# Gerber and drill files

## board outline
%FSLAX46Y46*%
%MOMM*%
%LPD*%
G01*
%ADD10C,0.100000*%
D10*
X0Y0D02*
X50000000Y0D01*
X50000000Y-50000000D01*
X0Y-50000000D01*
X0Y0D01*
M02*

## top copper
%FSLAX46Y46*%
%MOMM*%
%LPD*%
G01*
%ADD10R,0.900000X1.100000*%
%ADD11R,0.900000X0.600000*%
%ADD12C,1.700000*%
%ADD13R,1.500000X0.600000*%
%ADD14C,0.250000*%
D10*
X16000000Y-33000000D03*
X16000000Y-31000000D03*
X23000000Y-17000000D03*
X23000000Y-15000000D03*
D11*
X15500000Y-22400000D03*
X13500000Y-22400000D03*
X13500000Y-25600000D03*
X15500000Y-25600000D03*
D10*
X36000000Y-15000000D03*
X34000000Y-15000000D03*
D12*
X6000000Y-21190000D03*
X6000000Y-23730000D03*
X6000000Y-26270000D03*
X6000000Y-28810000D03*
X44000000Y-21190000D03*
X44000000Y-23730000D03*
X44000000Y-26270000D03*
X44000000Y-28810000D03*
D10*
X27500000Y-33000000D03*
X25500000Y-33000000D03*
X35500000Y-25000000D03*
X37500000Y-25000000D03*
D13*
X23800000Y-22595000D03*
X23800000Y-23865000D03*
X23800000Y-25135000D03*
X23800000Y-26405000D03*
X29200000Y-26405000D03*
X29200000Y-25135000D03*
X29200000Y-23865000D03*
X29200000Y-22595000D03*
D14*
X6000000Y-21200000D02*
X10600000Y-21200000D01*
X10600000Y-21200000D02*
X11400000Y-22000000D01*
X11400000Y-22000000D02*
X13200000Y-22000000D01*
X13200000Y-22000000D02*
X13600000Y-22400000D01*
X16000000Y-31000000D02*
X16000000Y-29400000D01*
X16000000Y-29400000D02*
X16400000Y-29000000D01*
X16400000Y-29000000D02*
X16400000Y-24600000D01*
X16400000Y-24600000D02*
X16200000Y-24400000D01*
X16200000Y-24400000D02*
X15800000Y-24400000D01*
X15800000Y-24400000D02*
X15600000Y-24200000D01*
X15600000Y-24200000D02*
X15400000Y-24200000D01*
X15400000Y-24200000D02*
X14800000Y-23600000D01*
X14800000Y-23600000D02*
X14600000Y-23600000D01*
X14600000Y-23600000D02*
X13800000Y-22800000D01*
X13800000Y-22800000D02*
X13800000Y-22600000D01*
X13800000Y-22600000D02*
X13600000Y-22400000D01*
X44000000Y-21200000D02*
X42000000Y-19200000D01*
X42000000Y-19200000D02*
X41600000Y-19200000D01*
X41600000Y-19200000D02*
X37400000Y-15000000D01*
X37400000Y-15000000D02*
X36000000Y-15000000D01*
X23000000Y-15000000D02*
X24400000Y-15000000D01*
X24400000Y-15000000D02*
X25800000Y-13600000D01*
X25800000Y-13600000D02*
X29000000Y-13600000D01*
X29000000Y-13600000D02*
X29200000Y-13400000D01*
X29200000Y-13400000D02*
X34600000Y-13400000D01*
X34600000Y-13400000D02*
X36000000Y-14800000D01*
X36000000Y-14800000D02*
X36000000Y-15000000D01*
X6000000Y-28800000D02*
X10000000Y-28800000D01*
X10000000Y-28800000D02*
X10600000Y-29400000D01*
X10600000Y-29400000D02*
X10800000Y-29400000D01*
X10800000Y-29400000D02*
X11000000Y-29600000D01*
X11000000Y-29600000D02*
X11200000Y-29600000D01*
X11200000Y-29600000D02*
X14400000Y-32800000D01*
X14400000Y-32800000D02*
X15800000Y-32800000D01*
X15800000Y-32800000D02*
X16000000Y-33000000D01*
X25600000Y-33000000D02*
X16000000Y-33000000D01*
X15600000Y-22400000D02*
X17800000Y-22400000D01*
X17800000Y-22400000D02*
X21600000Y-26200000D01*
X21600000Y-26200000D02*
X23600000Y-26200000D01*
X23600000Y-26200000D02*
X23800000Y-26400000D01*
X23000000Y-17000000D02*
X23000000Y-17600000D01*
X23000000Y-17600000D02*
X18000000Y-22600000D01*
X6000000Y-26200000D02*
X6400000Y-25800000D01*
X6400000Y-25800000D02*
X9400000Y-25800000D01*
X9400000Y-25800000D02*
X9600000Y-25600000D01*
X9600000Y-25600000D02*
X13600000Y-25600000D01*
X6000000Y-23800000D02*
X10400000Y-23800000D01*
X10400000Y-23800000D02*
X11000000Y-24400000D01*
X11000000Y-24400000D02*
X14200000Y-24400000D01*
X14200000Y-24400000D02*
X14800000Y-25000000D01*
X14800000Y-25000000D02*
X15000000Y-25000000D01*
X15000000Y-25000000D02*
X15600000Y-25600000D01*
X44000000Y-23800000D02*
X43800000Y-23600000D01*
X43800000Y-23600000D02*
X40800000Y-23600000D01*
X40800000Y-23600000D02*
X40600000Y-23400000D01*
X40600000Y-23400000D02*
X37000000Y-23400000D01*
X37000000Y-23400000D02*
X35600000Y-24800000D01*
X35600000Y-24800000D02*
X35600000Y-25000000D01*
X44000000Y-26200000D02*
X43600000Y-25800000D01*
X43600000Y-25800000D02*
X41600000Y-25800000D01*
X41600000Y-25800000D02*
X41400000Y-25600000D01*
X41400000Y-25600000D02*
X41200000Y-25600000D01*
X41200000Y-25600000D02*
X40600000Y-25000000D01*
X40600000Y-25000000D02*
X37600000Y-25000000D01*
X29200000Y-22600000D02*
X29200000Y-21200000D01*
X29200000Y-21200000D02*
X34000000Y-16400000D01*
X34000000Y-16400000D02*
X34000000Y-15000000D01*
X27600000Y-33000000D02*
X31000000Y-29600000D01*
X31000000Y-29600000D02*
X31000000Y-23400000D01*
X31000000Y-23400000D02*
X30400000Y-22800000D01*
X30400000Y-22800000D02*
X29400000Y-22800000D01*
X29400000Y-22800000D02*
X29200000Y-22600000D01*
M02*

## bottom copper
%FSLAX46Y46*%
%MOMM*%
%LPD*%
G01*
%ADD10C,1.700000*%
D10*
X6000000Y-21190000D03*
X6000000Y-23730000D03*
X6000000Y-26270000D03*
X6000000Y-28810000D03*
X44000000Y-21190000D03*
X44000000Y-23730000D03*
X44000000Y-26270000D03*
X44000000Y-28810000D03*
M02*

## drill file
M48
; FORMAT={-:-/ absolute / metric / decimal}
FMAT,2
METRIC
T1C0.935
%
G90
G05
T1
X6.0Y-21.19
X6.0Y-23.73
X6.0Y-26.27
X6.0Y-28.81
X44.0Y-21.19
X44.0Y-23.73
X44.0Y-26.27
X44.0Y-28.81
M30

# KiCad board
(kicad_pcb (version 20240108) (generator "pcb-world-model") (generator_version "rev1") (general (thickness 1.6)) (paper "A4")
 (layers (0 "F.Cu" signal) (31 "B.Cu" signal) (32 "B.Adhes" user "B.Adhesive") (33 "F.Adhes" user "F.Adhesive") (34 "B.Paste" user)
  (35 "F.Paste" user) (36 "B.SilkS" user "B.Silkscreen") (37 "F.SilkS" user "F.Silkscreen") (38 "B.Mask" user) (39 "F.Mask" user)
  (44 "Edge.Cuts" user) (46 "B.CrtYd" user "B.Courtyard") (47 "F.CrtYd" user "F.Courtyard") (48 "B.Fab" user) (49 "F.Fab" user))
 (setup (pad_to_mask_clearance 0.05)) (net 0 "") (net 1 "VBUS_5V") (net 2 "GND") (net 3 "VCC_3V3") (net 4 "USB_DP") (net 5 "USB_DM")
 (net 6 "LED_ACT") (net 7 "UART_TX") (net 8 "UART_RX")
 (gr_rect (start 0.0 0.0) (end 50.0000 50.0000) (stroke (width 0.1) (type default)) (fill none) (layer "Edge.Cuts"))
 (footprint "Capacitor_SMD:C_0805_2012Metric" (layer "F.Cu") (at 16.0000 32.0000 90)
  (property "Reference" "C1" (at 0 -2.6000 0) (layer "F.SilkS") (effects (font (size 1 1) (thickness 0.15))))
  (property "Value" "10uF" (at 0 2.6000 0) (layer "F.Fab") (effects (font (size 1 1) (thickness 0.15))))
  (pad "1" smd rect (at -1.0000 0.0000) (size 0.9000 1.1000) (layers "F.Cu" "F.Paste" "F.Mask") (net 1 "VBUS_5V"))
  (pad "2" smd rect (at 1.0000 0.0000) (size 0.9000 1.1000) (layers "F.Cu" "F.Paste" "F.Mask") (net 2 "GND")))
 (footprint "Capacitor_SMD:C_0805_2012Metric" (layer "F.Cu") (at 23.0000 16.0000 90)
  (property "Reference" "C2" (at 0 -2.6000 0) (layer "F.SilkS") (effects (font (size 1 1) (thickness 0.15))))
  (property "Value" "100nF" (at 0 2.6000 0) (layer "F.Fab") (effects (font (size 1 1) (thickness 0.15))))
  (pad "1" smd rect (at -1.0000 0.0000) (size 0.9000 1.1000) (layers "F.Cu" "F.Paste" "F.Mask") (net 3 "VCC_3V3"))
  (pad "2" smd rect (at 1.0000 0.0000) (size 0.9000 1.1000) (layers "F.Cu" "F.Paste" "F.Mask") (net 2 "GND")))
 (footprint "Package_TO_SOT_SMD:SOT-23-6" (layer "F.Cu") (at 14.5000 24.0000 270)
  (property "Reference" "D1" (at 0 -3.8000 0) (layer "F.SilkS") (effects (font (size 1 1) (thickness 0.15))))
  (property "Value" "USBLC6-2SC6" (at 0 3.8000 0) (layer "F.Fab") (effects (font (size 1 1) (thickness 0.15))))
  (pad "1" smd rect (at -1.6000 -1.0000) (size 0.9000 0.6000) (layers "F.Cu" "F.Paste" "F.Mask") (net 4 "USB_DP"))
  (pad "2" smd rect (at -1.6000 1.0000) (size 0.9000 0.6000) (layers "F.Cu" "F.Paste" "F.Mask") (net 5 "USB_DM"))
  (pad "3" smd rect (at 1.6000 1.0000) (size 0.9000 0.6000) (layers "F.Cu" "F.Paste" "F.Mask") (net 2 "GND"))
  (pad "4" smd rect (at 1.6000 -1.0000) (size 0.9000 0.6000) (layers "F.Cu" "F.Paste" "F.Mask") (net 1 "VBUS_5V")))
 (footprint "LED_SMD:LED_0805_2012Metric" (layer "F.Cu") (at 35.0000 15.0000 180)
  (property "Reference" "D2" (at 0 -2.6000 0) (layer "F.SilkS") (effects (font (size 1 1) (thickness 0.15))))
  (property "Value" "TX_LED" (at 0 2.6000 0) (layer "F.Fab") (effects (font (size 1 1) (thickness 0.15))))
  (pad "1" smd rect (at -1.0000 0.0000) (size 0.9000 1.1000) (layers "F.Cu" "F.Paste" "F.Mask") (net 3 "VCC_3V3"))
  (pad "2" smd rect (at 1.0000 0.0000) (size 0.9000 1.1000) (layers "F.Cu" "F.Paste" "F.Mask") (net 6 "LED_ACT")))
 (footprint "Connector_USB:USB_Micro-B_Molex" (layer "F.Cu") (at 6.0000 25.0000 0) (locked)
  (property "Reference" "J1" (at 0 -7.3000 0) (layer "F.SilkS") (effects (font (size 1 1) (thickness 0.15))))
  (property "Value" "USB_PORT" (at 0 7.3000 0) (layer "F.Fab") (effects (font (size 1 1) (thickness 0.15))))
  (pad "1" thru_hole circle (at 0.0000 -3.8100) (size 1.7000 1.7000) (drill 0.9350) (layers "*.Cu" "*.Mask") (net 1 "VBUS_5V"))
  (pad "2" thru_hole circle (at 0.0000 -1.2700) (size 1.7000 1.7000) (drill 0.9350) (layers "*.Cu" "*.Mask") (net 5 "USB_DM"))
  (pad "3" thru_hole circle (at 0.0000 1.2700) (size 1.7000 1.7000) (drill 0.9350) (layers "*.Cu" "*.Mask") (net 4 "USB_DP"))
  (pad "4" thru_hole circle (at 0.0000 3.8100) (size 1.7000 1.7000) (drill 0.9350) (layers "*.Cu" "*.Mask") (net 2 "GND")))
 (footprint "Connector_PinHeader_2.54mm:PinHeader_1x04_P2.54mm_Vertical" (layer "F.Cu") (at 44.0000 25.0000 0) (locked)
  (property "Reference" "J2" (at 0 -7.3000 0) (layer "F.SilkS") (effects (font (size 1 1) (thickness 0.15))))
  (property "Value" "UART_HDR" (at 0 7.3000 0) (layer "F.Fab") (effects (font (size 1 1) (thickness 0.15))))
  (pad "1" thru_hole circle (at 0.0000 -3.8100) (size 1.7000 1.7000) (drill 0.9350) (layers "*.Cu" "*.Mask") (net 3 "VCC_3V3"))
  (pad "2" thru_hole circle (at 0.0000 -1.2700) (size 1.7000 1.7000) (drill 0.9350) (layers "*.Cu" "*.Mask") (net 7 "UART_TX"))
  (pad "3" thru_hole circle (at 0.0000 1.2700) (size 1.7000 1.7000) (drill 0.9350) (layers "*.Cu" "*.Mask") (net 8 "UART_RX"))
  (pad "4" thru_hole circle (at 0.0000 3.8100) (size 1.7000 1.7000) (drill 0.9350) (layers "*.Cu" "*.Mask") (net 2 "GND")))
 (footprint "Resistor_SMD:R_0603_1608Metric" (layer "F.Cu") (at 26.5000 33.0000 180)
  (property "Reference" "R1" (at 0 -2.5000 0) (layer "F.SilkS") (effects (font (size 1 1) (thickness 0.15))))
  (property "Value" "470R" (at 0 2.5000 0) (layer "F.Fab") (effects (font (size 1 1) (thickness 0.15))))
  (pad "1" smd rect (at -1.0000 0.0000) (size 0.9000 1.1000) (layers "F.Cu" "F.Paste" "F.Mask") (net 6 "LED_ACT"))
  (pad "2" smd rect (at 1.0000 0.0000) (size 0.9000 1.1000) (layers "F.Cu" "F.Paste" "F.Mask") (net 2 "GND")))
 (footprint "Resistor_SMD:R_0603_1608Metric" (layer "F.Cu") (at 36.5000 25.0000 0)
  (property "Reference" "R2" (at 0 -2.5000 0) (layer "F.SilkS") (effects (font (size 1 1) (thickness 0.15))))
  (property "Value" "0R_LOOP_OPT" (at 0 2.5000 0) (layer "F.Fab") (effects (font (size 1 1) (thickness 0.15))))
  (pad "1" smd rect (at -1.0000 0.0000) (size 0.9000 1.1000) (layers "F.Cu" "F.Paste" "F.Mask") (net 7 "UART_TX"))
  (pad "2" smd rect (at 1.0000 0.0000) (size 0.9000 1.1000) (layers "F.Cu" "F.Paste" "F.Mask") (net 8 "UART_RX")))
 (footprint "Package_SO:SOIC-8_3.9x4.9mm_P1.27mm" (layer "F.Cu") (at 26.5000 24.5000 0)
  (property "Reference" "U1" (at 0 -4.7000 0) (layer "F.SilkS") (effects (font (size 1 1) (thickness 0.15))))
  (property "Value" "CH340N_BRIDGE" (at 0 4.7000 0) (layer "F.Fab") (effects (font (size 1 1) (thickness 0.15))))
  (pad "1" smd rect (at -2.7000 -1.9050) (size 1.5000 0.6000) (layers "F.Cu" "F.Paste" "F.Mask") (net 1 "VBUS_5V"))
  (pad "2" smd rect (at -2.7000 -0.6350) (size 1.5000 0.6000) (layers "F.Cu" "F.Paste" "F.Mask") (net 4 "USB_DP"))
  (pad "3" smd rect (at -2.7000 0.6350) (size 1.5000 0.6000) (layers "F.Cu" "F.Paste" "F.Mask") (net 5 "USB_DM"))
  (pad "4" smd rect (at -2.7000 1.9050) (size 1.5000 0.6000) (layers "F.Cu" "F.Paste" "F.Mask") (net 2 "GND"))
  (pad "5" smd rect (at 2.7000 1.9050) (size 1.5000 0.6000) (layers "F.Cu" "F.Paste" "F.Mask") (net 3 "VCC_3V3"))
  (pad "6" smd rect (at 2.7000 0.6350) (size 1.5000 0.6000) (layers "F.Cu" "F.Paste" "F.Mask") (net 7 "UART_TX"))
  (pad "7" smd rect (at 2.7000 -0.6350) (size 1.5000 0.6000) (layers "F.Cu" "F.Paste" "F.Mask") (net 8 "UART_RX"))
  (pad "8" smd rect (at 2.7000 -1.9050) (size 1.5000 0.6000) (layers "F.Cu" "F.Paste" "F.Mask") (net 6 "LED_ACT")))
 (segment (start 6.0000 21.2000) (end 10.6000 21.2000) (width 0.2500) (layer "F.Cu") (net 1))
 (segment (start 10.6000 21.2000) (end 11.4000 22.0000) (width 0.2500) (layer "F.Cu") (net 1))
 (segment (start 11.4000 22.0000) (end 13.2000 22.0000) (width 0.2500) (layer "F.Cu") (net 1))
 (segment (start 13.2000 22.0000) (end 13.6000 22.4000) (width 0.2500) (layer "F.Cu") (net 1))
 (segment (start 16.0000 31.0000) (end 16.0000 29.4000) (width 0.2500) (layer "F.Cu") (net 1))
 (segment (start 16.0000 29.4000) (end 16.4000 29.0000) (width 0.2500) (layer "F.Cu") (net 1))
 (segment (start 16.4000 29.0000) (end 16.4000 24.6000) (width 0.2500) (layer "F.Cu") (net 1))
 (segment (start 16.4000 24.6000) (end 16.2000 24.4000) (width 0.2500) (layer "F.Cu") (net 1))
 (segment (start 16.2000 24.4000) (end 15.8000 24.4000) (width 0.2500) (layer "F.Cu") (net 1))
 (segment (start 15.8000 24.4000) (end 15.6000 24.2000) (width 0.2500) (layer "F.Cu") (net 1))
 (segment (start 15.6000 24.2000) (end 15.4000 24.2000) (width 0.2500) (layer "F.Cu") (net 1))
 (segment (start 15.4000 24.2000) (end 14.8000 23.6000) (width 0.2500) (layer "F.Cu") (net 1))
 (segment (start 14.8000 23.6000) (end 14.6000 23.6000) (width 0.2500) (layer "F.Cu") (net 1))
 (segment (start 14.6000 23.6000) (end 13.8000 22.8000) (width 0.2500) (layer "F.Cu") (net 1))
 (segment (start 13.8000 22.8000) (end 13.8000 22.6000) (width 0.2500) (layer "F.Cu") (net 1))
 (segment (start 13.8000 22.6000) (end 13.6000 22.4000) (width 0.2500) (layer "F.Cu") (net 1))
 (segment (start 44.0000 21.2000) (end 42.0000 19.2000) (width 0.2500) (layer "F.Cu") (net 3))
 (segment (start 42.0000 19.2000) (end 41.6000 19.2000) (width 0.2500) (layer "F.Cu") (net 3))
 (segment (start 41.6000 19.2000) (end 37.4000 15.0000) (width 0.2500) (layer "F.Cu") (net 3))
 (segment (start 37.4000 15.0000) (end 36.0000 15.0000) (width 0.2500) (layer "F.Cu") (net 3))
 (segment (start 23.0000 15.0000) (end 24.4000 15.0000) (width 0.2500) (layer "F.Cu") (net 3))
 (segment (start 24.4000 15.0000) (end 25.8000 13.6000) (width 0.2500) (layer "F.Cu") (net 3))
 (segment (start 25.8000 13.6000) (end 29.0000 13.6000) (width 0.2500) (layer "F.Cu") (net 3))
 (segment (start 29.0000 13.6000) (end 29.2000 13.4000) (width 0.2500) (layer "F.Cu") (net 3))
 (segment (start 29.2000 13.4000) (end 34.6000 13.4000) (width 0.2500) (layer "F.Cu") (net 3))
 (segment (start 34.6000 13.4000) (end 36.0000 14.8000) (width 0.2500) (layer "F.Cu") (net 3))
 (segment (start 36.0000 14.8000) (end 36.0000 15.0000) (width 0.2500) (layer "F.Cu") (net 3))
 (segment (start 6.0000 28.8000) (end 10.0000 28.8000) (width 0.2500) (layer "F.Cu") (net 2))
 (segment (start 10.0000 28.8000) (end 10.6000 29.4000) (width 0.2500) (layer "F.Cu") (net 2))
 (segment (start 10.6000 29.4000) (end 10.8000 29.4000) (width 0.2500) (layer "F.Cu") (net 2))
 (segment (start 10.8000 29.4000) (end 11.0000 29.6000) (width 0.2500) (layer "F.Cu") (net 2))
 (segment (start 11.0000 29.6000) (end 11.2000 29.6000) (width 0.2500) (layer "F.Cu") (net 2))
 (segment (start 11.2000 29.6000) (end 14.4000 32.8000) (width 0.2500) (layer "F.Cu") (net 2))
 (segment (start 14.4000 32.8000) (end 15.8000 32.8000) (width 0.2500) (layer "F.Cu") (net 2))
 (segment (start 15.8000 32.8000) (end 16.0000 33.0000) (width 0.2500) (layer "F.Cu") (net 2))
 (segment (start 25.6000 33.0000) (end 16.0000 33.0000) (width 0.2500) (layer "F.Cu") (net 2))
 (segment (start 15.6000 22.4000) (end 17.8000 22.4000) (width 0.2500) (layer "F.Cu") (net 2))
 (segment (start 17.8000 22.4000) (end 21.6000 26.2000) (width 0.2500) (layer "F.Cu") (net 2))
 (segment (start 21.6000 26.2000) (end 23.6000 26.2000) (width 0.2500) (layer "F.Cu") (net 2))
 (segment (start 23.6000 26.2000) (end 23.8000 26.4000) (width 0.2500) (layer "F.Cu") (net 2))
 (segment (start 23.0000 17.0000) (end 23.0000 17.6000) (width 0.2500) (layer "F.Cu") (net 2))
 (segment (start 23.0000 17.6000) (end 18.0000 22.6000) (width 0.2500) (layer "F.Cu") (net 2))
 (segment (start 6.0000 26.2000) (end 6.4000 25.8000) (width 0.2500) (layer "F.Cu") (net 4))
 (segment (start 6.4000 25.8000) (end 9.4000 25.8000) (width 0.2500) (layer "F.Cu") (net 4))
 (segment (start 9.4000 25.8000) (end 9.6000 25.6000) (width 0.2500) (layer "F.Cu") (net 4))
 (segment (start 9.6000 25.6000) (end 13.6000 25.6000) (width 0.2500) (layer "F.Cu") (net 4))
 (segment (start 6.0000 23.8000) (end 10.4000 23.8000) (width 0.2500) (layer "F.Cu") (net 5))
 (segment (start 10.4000 23.8000) (end 11.0000 24.4000) (width 0.2500) (layer "F.Cu") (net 5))
 (segment (start 11.0000 24.4000) (end 14.2000 24.4000) (width 0.2500) (layer "F.Cu") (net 5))
 (segment (start 14.2000 24.4000) (end 14.8000 25.0000) (width 0.2500) (layer "F.Cu") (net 5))
 (segment (start 14.8000 25.0000) (end 15.0000 25.0000) (width 0.2500) (layer "F.Cu") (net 5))
 (segment (start 15.0000 25.0000) (end 15.6000 25.6000) (width 0.2500) (layer "F.Cu") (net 5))
 (segment (start 44.0000 23.8000) (end 43.8000 23.6000) (width 0.2500) (layer "F.Cu") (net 7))
 (segment (start 43.8000 23.6000) (end 40.8000 23.6000) (width 0.2500) (layer "F.Cu") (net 7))
 (segment (start 40.8000 23.6000) (end 40.6000 23.4000) (width 0.2500) (layer "F.Cu") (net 7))
 (segment (start 40.6000 23.4000) (end 37.0000 23.4000) (width 0.2500) (layer "F.Cu") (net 7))
 (segment (start 37.0000 23.4000) (end 35.6000 24.8000) (width 0.2500) (layer "F.Cu") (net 7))
 (segment (start 35.6000 24.8000) (end 35.6000 25.0000) (width 0.2500) (layer "F.Cu") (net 7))
 (segment (start 44.0000 26.2000) (end 43.6000 25.8000) (width 0.2500) (layer "F.Cu") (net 8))
 (segment (start 43.6000 25.8000) (end 41.6000 25.8000) (width 0.2500) (layer "F.Cu") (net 8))
 (segment (start 41.6000 25.8000) (end 41.4000 25.6000) (width 0.2500) (layer "F.Cu") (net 8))
 (segment (start 41.4000 25.6000) (end 41.2000 25.6000) (width 0.2500) (layer "F.Cu") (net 8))
 (segment (start 41.2000 25.6000) (end 40.6000 25.0000) (width 0.2500) (layer "F.Cu") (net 8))
 (segment (start 40.6000 25.0000) (end 37.6000 25.0000) (width 0.2500) (layer "F.Cu") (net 8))
 (segment (start 29.2000 22.6000) (end 29.2000 21.2000) (width 0.2500) (layer "F.Cu") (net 6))
 (segment (start 29.2000 21.2000) (end 34.0000 16.4000) (width 0.2500) (layer "F.Cu") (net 6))
 (segment (start 34.0000 16.4000) (end 34.0000 15.0000) (width 0.2500) (layer "F.Cu") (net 6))
 (segment (start 27.6000 33.0000) (end 31.0000 29.6000) (width 0.2500) (layer "F.Cu") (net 6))
 (segment (start 31.0000 29.6000) (end 31.0000 23.4000) (width 0.2500) (layer "F.Cu") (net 6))
 (segment (start 31.0000 23.4000) (end 30.4000 22.8000) (width 0.2500) (layer "F.Cu") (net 6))
 (segment (start 30.4000 22.8000) (end 29.4000 22.8000) (width 0.2500) (layer "F.Cu") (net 6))
 (segment (start 29.4000 22.8000) (end 29.2000 22.6000) (width 0.2500) (layer "F.Cu") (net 6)))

